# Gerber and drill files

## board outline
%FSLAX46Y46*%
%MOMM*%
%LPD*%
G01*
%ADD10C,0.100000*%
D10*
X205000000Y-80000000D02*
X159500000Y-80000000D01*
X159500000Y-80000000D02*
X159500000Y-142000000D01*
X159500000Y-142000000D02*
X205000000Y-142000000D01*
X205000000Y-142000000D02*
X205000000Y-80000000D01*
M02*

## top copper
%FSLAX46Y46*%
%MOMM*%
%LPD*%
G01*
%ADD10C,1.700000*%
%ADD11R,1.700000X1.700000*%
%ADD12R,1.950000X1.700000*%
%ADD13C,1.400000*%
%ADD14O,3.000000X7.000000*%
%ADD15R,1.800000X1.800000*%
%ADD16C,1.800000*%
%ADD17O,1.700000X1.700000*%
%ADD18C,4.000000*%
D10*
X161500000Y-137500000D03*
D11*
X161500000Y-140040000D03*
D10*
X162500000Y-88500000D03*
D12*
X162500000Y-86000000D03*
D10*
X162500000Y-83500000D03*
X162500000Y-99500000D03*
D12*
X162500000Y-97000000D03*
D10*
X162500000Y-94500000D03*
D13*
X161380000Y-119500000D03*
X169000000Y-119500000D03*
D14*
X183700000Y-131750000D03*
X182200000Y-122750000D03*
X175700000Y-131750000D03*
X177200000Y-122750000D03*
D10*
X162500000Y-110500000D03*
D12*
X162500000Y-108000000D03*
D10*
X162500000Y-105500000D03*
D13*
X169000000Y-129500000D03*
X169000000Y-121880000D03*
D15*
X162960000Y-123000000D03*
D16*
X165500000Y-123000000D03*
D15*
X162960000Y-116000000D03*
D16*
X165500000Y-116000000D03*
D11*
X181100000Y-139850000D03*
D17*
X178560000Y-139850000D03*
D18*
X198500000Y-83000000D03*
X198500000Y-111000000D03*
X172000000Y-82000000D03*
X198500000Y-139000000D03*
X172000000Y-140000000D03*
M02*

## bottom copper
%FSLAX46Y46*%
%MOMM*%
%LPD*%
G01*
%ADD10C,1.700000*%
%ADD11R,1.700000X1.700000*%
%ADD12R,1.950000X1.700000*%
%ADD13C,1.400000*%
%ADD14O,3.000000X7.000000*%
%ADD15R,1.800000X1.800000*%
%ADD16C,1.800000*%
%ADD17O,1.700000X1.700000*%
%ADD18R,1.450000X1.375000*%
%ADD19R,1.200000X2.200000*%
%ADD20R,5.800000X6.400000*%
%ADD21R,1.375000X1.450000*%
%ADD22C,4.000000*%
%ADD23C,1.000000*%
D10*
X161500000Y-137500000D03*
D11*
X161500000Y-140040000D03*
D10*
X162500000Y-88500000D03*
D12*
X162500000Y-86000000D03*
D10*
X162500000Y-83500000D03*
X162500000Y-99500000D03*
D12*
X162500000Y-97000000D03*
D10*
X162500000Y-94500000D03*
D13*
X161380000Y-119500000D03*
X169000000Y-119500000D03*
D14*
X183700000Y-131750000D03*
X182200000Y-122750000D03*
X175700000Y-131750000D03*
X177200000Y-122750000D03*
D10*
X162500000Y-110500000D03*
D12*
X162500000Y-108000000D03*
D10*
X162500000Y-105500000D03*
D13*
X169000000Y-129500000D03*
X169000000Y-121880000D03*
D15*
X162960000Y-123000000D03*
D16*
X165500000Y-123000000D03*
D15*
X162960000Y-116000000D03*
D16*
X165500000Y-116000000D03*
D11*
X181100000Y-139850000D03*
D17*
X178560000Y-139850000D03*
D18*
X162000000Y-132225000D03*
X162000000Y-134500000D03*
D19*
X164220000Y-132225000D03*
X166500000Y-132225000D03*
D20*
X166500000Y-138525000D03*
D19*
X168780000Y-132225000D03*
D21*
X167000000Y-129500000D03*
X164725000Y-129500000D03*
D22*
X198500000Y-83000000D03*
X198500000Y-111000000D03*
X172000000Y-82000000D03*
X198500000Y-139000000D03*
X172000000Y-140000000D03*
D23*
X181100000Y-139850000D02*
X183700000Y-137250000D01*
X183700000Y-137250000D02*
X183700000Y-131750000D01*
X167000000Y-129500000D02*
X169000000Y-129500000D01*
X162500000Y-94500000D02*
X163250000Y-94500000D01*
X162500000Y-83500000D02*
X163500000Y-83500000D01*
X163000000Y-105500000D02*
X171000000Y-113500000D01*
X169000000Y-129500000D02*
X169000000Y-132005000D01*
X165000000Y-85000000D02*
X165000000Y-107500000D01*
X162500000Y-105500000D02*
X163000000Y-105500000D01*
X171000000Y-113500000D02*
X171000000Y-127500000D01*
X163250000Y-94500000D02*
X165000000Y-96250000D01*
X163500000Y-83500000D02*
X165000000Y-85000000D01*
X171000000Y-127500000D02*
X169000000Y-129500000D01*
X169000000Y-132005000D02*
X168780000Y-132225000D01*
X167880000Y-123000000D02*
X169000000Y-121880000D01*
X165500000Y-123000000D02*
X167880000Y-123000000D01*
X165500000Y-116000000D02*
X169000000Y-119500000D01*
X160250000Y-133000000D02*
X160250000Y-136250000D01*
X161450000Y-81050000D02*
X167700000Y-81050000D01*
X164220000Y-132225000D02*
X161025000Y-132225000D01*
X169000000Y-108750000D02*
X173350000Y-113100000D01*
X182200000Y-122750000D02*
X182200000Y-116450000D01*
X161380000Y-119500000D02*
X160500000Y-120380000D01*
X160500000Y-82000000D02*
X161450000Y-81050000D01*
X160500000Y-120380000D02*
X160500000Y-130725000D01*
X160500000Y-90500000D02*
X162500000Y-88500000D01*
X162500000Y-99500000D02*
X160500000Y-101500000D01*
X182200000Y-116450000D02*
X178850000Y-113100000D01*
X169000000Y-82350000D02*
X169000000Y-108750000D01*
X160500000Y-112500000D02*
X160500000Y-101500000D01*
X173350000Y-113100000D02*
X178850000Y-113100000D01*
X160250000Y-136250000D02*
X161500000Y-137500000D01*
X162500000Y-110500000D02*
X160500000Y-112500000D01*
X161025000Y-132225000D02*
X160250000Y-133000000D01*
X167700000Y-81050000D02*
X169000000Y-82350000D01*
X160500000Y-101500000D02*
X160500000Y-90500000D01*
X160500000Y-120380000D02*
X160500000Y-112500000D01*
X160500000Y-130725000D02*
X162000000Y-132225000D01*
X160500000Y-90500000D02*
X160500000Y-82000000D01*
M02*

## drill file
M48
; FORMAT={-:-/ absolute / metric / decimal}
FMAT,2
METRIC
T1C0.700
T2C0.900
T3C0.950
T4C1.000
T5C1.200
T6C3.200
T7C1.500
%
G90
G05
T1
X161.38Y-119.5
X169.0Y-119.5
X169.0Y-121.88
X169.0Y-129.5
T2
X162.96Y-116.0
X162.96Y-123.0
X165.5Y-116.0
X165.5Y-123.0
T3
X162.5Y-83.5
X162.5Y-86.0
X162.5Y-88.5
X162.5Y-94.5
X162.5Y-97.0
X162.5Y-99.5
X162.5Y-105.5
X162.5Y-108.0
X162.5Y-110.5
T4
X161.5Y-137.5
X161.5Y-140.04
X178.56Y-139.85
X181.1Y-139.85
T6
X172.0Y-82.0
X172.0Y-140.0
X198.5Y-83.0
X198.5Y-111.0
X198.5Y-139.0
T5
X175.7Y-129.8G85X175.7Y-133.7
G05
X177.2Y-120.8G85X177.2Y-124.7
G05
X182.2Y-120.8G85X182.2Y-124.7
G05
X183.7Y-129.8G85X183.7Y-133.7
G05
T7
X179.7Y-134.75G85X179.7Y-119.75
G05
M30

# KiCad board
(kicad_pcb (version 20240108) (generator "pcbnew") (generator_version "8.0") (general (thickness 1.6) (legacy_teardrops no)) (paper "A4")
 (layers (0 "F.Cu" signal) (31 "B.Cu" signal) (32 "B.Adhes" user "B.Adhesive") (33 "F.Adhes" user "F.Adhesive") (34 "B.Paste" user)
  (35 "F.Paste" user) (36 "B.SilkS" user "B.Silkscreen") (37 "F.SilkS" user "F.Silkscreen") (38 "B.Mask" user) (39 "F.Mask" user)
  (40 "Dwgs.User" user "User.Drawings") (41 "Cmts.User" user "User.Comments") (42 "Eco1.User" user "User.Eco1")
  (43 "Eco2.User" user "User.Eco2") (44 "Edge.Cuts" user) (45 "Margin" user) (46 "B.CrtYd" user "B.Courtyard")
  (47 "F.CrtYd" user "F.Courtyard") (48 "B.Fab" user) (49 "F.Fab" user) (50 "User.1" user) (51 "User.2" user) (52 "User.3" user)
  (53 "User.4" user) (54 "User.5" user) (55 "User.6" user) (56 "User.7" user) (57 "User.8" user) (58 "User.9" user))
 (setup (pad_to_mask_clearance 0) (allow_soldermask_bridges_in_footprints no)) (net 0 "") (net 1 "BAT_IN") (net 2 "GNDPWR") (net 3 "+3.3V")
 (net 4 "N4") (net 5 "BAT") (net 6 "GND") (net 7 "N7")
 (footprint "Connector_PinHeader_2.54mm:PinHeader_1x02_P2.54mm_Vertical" (layer "F.Cu") (at 161.5 137.5)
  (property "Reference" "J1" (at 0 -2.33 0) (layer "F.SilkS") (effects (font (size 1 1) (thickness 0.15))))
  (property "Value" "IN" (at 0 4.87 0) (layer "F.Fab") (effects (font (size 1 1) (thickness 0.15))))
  (pad "1" thru_hole circle (at 0 0) (size 1.7 1.7) (drill 1) (layers "*.Cu" "*.Mask") (remove_unused_layers no) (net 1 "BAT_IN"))
  (pad "2" thru_hole rect (at 0 2.54) (size 1.7 1.7) (drill 1) (layers "*.Cu" "*.Mask") (remove_unused_layers no) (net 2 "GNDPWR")))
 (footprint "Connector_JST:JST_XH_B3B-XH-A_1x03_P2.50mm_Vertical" (layer "F.Cu") (at 162.5 88.5 90)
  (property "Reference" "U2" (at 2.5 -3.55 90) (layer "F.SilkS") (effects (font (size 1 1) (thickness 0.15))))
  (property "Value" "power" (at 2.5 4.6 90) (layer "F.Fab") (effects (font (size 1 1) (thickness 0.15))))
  (pad "1" thru_hole circle (at 0 0 90) (size 1.7 1.7) (drill 0.95) (layers "*.Cu" "*.Mask" "Dwgs.User") (remove_unused_layers no)
   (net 1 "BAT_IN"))
  (pad "2" thru_hole rect (at 2.5 0 90) (size 1.7 1.95) (drill 0.95) (layers "*.Cu" "*.Mask") (remove_unused_layers no) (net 2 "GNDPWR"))
  (pad "3" thru_hole circle (at 5 0 90) (size 1.7 1.7) (drill 0.95) (layers "*.Cu" "*.Mask") (remove_unused_layers no) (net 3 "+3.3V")))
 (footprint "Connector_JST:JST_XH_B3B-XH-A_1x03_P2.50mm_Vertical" (layer "F.Cu") (at 162.5 99.5 90)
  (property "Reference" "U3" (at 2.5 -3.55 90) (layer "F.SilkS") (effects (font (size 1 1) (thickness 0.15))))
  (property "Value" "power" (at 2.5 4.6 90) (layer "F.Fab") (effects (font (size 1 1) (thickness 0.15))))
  (pad "1" thru_hole circle (at 0 0 90) (size 1.7 1.7) (drill 0.95) (layers "*.Cu" "*.Mask") (remove_unused_layers no) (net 1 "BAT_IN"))
  (pad "2" thru_hole rect (at 2.5 0 90) (size 1.7 1.95) (drill 0.95) (layers "*.Cu" "*.Mask") (remove_unused_layers no) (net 2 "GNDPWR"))
  (pad "3" thru_hole circle (at 5 0 90) (size 1.7 1.7) (drill 0.95) (layers "*.Cu" "*.Mask") (remove_unused_layers no) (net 3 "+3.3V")))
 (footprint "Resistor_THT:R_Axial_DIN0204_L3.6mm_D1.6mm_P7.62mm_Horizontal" (layer "F.Cu") (at 161.38 119.5)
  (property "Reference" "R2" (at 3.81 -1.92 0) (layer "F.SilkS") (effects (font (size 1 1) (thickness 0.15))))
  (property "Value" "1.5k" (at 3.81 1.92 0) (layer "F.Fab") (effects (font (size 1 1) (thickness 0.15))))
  (pad "1" thru_hole circle (at 0 0) (size 1.4 1.4) (drill 0.7) (layers "*.Cu" "*.Mask") (remove_unused_layers no) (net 1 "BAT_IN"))
  (pad "2" thru_hole circle (at 7.62 0) (size 1.4 1.4) (drill 0.7) (layers "*.Cu" "*.Mask") (remove_unused_layers no) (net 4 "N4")))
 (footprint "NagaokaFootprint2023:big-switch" (layer "F.Cu") (at 179.7 125.75 180)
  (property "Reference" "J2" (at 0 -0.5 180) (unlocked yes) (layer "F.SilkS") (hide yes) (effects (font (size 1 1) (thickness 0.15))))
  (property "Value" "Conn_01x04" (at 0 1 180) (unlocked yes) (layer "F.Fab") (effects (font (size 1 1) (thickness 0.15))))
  (pad "" np_thru_hole circle (at 0 -1.5 180) (size 1 1) (drill oval 1.5 16.5) (layers "F&B.Cu" "*.Mask"))
  (pad "1" thru_hole oval (at -4 -6 270) (size 7 3) (drill oval 5.1 1.2) (layers "*.Cu" "*.Mask") (remove_unused_layers no) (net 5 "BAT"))
  (pad "2" thru_hole oval (at -2.5 3 270) (size 7 3) (drill oval 5.1 1.2) (layers "*.Cu" "*.Mask") (remove_unused_layers no)
   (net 1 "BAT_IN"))
  (pad "3" thru_hole oval (at 4 -6 270) (size 7 3) (drill oval 5.1 1.2) (layers "*.Cu" "*.Mask") (remove_unused_layers no) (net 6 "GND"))
  (pad "4" thru_hole oval (at 2.5 3 270) (size 7 3) (drill oval 5.1 1.2) (layers "*.Cu" "*.Mask") (remove_unused_layers no) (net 2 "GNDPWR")))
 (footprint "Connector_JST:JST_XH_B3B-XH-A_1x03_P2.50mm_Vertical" (layer "F.Cu") (at 162.5 110.5 90)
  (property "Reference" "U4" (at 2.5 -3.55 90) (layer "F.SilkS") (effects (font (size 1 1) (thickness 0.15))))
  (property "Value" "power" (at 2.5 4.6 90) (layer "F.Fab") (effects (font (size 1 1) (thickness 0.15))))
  (pad "1" thru_hole circle (at 0 0 90) (size 1.7 1.7) (drill 0.95) (layers "*.Cu" "*.Mask") (remove_unused_layers no) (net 1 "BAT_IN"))
  (pad "2" thru_hole rect (at 2.5 0 90) (size 1.7 1.95) (drill 0.95) (layers "*.Cu" "*.Mask") (remove_unused_layers no) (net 2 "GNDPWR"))
  (pad "3" thru_hole circle (at 5 0 90) (size 1.7 1.7) (drill 0.95) (layers "*.Cu" "*.Mask") (remove_unused_layers no) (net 3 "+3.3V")))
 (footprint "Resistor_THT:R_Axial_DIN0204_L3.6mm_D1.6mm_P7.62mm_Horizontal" (layer "F.Cu") (at 169 129.5 90)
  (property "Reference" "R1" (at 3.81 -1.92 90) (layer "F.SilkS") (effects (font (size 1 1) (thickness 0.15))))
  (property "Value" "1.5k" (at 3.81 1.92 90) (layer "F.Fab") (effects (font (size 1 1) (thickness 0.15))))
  (pad "1" thru_hole circle (at 0 0 90) (size 1.4 1.4) (drill 0.7) (layers "*.Cu" "*.Mask") (remove_unused_layers no) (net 3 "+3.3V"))
  (pad "2" thru_hole circle (at 7.62 0 90) (size 1.4 1.4) (drill 0.7) (layers "*.Cu" "*.Mask") (remove_unused_layers no) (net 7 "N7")))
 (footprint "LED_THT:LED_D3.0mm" (layer "F.Cu") (at 162.96 123)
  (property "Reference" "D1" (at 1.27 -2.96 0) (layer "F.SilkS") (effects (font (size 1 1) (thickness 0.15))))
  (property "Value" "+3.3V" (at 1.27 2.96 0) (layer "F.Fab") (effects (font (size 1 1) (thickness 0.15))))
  (pad "1" thru_hole rect (at 0 0) (size 1.8 1.8) (drill 0.9) (layers "*.Cu" "*.Mask") (remove_unused_layers no) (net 2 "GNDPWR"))
  (pad "2" thru_hole circle (at 2.54 0) (size 1.8 1.8) (drill 0.9) (layers "*.Cu" "*.Mask") (remove_unused_layers no) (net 7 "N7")))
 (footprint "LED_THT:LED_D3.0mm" (layer "F.Cu") (at 162.96 116)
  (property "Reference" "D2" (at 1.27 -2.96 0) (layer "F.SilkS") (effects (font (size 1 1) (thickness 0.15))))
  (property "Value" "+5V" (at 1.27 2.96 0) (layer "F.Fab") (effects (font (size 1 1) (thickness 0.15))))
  (pad "1" thru_hole rect (at 0 0) (size 1.8 1.8) (drill 0.9) (layers "*.Cu" "*.Mask") (remove_unused_layers no) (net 2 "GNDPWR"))
  (pad "2" thru_hole circle (at 2.54 0) (size 1.8 1.8) (drill 0.9) (layers "*.Cu" "*.Mask") (remove_unused_layers no) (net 4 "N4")))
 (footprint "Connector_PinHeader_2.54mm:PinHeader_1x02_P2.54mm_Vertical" (layer "F.Cu") (at 181.1 139.85 -90)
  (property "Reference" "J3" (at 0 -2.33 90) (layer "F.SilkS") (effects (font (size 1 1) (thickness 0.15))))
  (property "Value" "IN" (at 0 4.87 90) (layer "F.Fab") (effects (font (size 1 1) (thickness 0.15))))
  (pad "1" thru_hole rect (at 0 0 270) (size 1.7 1.7) (drill 1) (layers "*.Cu" "*.Mask") (remove_unused_layers no) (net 5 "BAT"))
  (pad "2" thru_hole oval (at 0 2.54 270) (size 1.7 1.7) (drill 1) (layers "*.Cu" "*.Mask") (remove_unused_layers no) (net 6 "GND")))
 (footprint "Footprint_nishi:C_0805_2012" (layer "B.Cu") (at 162 133.3625 -90)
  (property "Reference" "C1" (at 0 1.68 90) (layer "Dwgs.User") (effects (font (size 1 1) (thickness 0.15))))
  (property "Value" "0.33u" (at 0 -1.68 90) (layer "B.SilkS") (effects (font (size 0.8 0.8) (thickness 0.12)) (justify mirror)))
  (pad "1" smd rect (at -1.1375 0 270) (size 1.375 1.45) (layers "B.Cu" "B.Paste" "B.Mask") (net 1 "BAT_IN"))
  (pad "2" smd rect (at 1.1375 0 270) (size 1.375 1.45) (layers "B.Cu" "B.Paste" "B.Mask") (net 2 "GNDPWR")))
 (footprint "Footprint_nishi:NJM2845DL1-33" (layer "B.Cu") (at 166.5 136.425 -90)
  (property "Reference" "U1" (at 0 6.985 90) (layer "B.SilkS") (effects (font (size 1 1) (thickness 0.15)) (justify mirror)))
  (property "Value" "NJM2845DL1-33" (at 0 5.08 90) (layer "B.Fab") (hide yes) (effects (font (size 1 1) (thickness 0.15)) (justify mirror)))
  (pad "1" smd rect (at -4.2 2.28 270) (size 2.2 1.2) (layers "B.Cu" "B.Paste" "B.Mask") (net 1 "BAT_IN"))
  (pad "2" smd rect (at -4.2 0 270) (size 2.2 1.2) (layers "B.Cu" "B.Paste" "B.Mask") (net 2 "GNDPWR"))
  (pad "2" smd rect (at 2.1 0 270) (size 6.4 5.8) (layers "B.Cu" "B.Paste" "B.Mask") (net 2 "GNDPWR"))
  (pad "3" smd rect (at -4.2 -2.28 270) (size 2.2 1.2) (layers "B.Cu" "B.Paste" "B.Mask") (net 3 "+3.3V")))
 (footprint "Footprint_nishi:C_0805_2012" (layer "B.Cu") (at 165.8625 129.5 180)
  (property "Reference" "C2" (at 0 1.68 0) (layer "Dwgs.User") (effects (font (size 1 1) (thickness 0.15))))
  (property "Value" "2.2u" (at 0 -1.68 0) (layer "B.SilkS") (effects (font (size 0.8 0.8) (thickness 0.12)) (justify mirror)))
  (pad "1" smd rect (at -1.1375 0 180) (size 1.375 1.45) (layers "B.Cu" "B.Paste" "B.Mask") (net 3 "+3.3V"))
  (pad "2" smd rect (at 1.1375 0 180) (size 1.375 1.45) (layers "B.Cu" "B.Paste" "B.Mask") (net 2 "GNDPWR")))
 (gr_line (start 205 80) (end 159.5 80) (stroke (width 0.1) (type default)) (layer "Edge.Cuts"))
 (gr_line (start 159.5 80) (end 159.5 142) (stroke (width 0.1) (type default)) (layer "Edge.Cuts"))
 (gr_line (start 159.5 142) (end 205 142) (stroke (width 0.1) (type default)) (layer "Edge.Cuts"))
 (gr_line (start 205 142) (end 205 80) (stroke (width 0.1) (type default)) (layer "Edge.Cuts"))
 (via (at 198.5 83) (size 4) (drill 3.2) (layers "F.Cu" "B.Cu") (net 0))
 (via (at 198.5 111) (size 4) (drill 3.2) (layers "F.Cu" "B.Cu") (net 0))
 (via (at 172 82) (size 4) (drill 3.2) (layers "F.Cu" "B.Cu") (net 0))
 (via (at 198.5 139) (size 4) (drill 3.2) (layers "F.Cu" "B.Cu") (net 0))
 (via (at 172 140) (size 4) (drill 3.2) (layers "F.Cu" "B.Cu") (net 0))
 (segment (start 181.1 139.85) (end 183.7 137.25) (width 1) (layer "B.Cu") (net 5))
 (segment (start 183.7 137.25) (end 183.7 131.75) (width 1) (layer "B.Cu") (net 5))
 (segment (start 167 129.5) (end 169 129.5) (width 1) (layer "B.Cu") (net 3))
 (segment (start 162.5 94.5) (end 163.25 94.5) (width 1) (layer "B.Cu") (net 3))
 (segment (start 162.5 83.5) (end 163.5 83.5) (width 1) (layer "B.Cu") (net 3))
 (segment (start 163 105.5) (end 171 113.5) (width 1) (layer "B.Cu") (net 3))
 (segment (start 169 129.5) (end 169 132.005) (width 1) (layer "B.Cu") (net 3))
 (segment (start 165 85) (end 165 107.5) (width 1) (layer "B.Cu") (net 3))
 (segment (start 162.5 105.5) (end 163 105.5) (width 1) (layer "B.Cu") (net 3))
 (segment (start 171 113.5) (end 171 127.5) (width 1) (layer "B.Cu") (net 3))
 (segment (start 163.25 94.5) (end 165 96.25) (width 1) (layer "B.Cu") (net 3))
 (segment (start 163.5 83.5) (end 165 85) (width 1) (layer "B.Cu") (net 3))
 (segment (start 171 127.5) (end 169 129.5) (width 1) (layer "B.Cu") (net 3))
 (segment (start 169 132.005) (end 168.78 132.225) (width 1) (layer "B.Cu") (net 3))
 (segment (start 167.88 123) (end 169 121.88) (width 1) (layer "B.Cu") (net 7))
 (segment (start 165.5 123) (end 167.88 123) (width 1) (layer "B.Cu") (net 7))
 (segment (start 165.5 116) (end 169 119.5) (width 1) (layer "B.Cu") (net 4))
 (segment (start 160.25 133) (end 160.25 136.25) (width 1) (layer "B.Cu") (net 1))
 (segment (start 161.45 81.05) (end 167.7 81.05) (width 1) (layer "B.Cu") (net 1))
 (segment (start 164.22 132.225) (end 161.025 132.225) (width 1) (layer "B.Cu") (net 1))
 (segment (start 169 108.75) (end 173.35 113.1) (width 1) (layer "B.Cu") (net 1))
 (segment (start 182.2 122.75) (end 182.2 116.45) (width 1) (layer "B.Cu") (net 1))
 (segment (start 161.38 119.5) (end 160.5 120.38) (width 1) (layer "B.Cu") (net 1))
 (segment (start 160.5 82) (end 161.45 81.05) (width 1) (layer "B.Cu") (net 1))
 (segment (start 160.5 120.38) (end 160.5 130.725) (width 1) (layer "B.Cu") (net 1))
 (segment (start 160.5 90.5) (end 162.5 88.5) (width 1) (layer "B.Cu") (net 1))
 (segment (start 162.5 99.5) (end 160.5 101.5) (width 1) (layer "B.Cu") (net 1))
 (segment (start 182.2 116.45) (end 178.85 113.1) (width 1) (layer "B.Cu") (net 1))
 (segment (start 169 82.35) (end 169 108.75) (width 1) (layer "B.Cu") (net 1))
 (segment (start 160.5 112.5) (end 160.5 101.5) (width 1) (layer "B.Cu") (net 1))
 (segment (start 173.35 113.1) (end 178.85 113.1) (width 1) (layer "B.Cu") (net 1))
 (segment (start 160.25 136.25) (end 161.5 137.5) (width 1) (layer "B.Cu") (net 1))
 (segment (start 162.5 110.5) (end 160.5 112.5) (width 1) (layer "B.Cu") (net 1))
 (segment (start 161.025 132.225) (end 160.25 133) (width 1) (layer "B.Cu") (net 1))
 (segment (start 167.7 81.05) (end 169 82.35) (width 1) (layer "B.Cu") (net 1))
 (segment (start 160.5 101.5) (end 160.5 90.5) (width 1) (layer "B.Cu") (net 1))
 (segment (start 160.5 120.38) (end 160.5 112.5) (width 1) (layer "B.Cu") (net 1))
 (segment (start 160.5 130.725) (end 162 132.225) (width 1) (layer "B.Cu") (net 1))
 (segment (start 160.5 90.5) (end 160.5 82) (width 1) (layer "B.Cu") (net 1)))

